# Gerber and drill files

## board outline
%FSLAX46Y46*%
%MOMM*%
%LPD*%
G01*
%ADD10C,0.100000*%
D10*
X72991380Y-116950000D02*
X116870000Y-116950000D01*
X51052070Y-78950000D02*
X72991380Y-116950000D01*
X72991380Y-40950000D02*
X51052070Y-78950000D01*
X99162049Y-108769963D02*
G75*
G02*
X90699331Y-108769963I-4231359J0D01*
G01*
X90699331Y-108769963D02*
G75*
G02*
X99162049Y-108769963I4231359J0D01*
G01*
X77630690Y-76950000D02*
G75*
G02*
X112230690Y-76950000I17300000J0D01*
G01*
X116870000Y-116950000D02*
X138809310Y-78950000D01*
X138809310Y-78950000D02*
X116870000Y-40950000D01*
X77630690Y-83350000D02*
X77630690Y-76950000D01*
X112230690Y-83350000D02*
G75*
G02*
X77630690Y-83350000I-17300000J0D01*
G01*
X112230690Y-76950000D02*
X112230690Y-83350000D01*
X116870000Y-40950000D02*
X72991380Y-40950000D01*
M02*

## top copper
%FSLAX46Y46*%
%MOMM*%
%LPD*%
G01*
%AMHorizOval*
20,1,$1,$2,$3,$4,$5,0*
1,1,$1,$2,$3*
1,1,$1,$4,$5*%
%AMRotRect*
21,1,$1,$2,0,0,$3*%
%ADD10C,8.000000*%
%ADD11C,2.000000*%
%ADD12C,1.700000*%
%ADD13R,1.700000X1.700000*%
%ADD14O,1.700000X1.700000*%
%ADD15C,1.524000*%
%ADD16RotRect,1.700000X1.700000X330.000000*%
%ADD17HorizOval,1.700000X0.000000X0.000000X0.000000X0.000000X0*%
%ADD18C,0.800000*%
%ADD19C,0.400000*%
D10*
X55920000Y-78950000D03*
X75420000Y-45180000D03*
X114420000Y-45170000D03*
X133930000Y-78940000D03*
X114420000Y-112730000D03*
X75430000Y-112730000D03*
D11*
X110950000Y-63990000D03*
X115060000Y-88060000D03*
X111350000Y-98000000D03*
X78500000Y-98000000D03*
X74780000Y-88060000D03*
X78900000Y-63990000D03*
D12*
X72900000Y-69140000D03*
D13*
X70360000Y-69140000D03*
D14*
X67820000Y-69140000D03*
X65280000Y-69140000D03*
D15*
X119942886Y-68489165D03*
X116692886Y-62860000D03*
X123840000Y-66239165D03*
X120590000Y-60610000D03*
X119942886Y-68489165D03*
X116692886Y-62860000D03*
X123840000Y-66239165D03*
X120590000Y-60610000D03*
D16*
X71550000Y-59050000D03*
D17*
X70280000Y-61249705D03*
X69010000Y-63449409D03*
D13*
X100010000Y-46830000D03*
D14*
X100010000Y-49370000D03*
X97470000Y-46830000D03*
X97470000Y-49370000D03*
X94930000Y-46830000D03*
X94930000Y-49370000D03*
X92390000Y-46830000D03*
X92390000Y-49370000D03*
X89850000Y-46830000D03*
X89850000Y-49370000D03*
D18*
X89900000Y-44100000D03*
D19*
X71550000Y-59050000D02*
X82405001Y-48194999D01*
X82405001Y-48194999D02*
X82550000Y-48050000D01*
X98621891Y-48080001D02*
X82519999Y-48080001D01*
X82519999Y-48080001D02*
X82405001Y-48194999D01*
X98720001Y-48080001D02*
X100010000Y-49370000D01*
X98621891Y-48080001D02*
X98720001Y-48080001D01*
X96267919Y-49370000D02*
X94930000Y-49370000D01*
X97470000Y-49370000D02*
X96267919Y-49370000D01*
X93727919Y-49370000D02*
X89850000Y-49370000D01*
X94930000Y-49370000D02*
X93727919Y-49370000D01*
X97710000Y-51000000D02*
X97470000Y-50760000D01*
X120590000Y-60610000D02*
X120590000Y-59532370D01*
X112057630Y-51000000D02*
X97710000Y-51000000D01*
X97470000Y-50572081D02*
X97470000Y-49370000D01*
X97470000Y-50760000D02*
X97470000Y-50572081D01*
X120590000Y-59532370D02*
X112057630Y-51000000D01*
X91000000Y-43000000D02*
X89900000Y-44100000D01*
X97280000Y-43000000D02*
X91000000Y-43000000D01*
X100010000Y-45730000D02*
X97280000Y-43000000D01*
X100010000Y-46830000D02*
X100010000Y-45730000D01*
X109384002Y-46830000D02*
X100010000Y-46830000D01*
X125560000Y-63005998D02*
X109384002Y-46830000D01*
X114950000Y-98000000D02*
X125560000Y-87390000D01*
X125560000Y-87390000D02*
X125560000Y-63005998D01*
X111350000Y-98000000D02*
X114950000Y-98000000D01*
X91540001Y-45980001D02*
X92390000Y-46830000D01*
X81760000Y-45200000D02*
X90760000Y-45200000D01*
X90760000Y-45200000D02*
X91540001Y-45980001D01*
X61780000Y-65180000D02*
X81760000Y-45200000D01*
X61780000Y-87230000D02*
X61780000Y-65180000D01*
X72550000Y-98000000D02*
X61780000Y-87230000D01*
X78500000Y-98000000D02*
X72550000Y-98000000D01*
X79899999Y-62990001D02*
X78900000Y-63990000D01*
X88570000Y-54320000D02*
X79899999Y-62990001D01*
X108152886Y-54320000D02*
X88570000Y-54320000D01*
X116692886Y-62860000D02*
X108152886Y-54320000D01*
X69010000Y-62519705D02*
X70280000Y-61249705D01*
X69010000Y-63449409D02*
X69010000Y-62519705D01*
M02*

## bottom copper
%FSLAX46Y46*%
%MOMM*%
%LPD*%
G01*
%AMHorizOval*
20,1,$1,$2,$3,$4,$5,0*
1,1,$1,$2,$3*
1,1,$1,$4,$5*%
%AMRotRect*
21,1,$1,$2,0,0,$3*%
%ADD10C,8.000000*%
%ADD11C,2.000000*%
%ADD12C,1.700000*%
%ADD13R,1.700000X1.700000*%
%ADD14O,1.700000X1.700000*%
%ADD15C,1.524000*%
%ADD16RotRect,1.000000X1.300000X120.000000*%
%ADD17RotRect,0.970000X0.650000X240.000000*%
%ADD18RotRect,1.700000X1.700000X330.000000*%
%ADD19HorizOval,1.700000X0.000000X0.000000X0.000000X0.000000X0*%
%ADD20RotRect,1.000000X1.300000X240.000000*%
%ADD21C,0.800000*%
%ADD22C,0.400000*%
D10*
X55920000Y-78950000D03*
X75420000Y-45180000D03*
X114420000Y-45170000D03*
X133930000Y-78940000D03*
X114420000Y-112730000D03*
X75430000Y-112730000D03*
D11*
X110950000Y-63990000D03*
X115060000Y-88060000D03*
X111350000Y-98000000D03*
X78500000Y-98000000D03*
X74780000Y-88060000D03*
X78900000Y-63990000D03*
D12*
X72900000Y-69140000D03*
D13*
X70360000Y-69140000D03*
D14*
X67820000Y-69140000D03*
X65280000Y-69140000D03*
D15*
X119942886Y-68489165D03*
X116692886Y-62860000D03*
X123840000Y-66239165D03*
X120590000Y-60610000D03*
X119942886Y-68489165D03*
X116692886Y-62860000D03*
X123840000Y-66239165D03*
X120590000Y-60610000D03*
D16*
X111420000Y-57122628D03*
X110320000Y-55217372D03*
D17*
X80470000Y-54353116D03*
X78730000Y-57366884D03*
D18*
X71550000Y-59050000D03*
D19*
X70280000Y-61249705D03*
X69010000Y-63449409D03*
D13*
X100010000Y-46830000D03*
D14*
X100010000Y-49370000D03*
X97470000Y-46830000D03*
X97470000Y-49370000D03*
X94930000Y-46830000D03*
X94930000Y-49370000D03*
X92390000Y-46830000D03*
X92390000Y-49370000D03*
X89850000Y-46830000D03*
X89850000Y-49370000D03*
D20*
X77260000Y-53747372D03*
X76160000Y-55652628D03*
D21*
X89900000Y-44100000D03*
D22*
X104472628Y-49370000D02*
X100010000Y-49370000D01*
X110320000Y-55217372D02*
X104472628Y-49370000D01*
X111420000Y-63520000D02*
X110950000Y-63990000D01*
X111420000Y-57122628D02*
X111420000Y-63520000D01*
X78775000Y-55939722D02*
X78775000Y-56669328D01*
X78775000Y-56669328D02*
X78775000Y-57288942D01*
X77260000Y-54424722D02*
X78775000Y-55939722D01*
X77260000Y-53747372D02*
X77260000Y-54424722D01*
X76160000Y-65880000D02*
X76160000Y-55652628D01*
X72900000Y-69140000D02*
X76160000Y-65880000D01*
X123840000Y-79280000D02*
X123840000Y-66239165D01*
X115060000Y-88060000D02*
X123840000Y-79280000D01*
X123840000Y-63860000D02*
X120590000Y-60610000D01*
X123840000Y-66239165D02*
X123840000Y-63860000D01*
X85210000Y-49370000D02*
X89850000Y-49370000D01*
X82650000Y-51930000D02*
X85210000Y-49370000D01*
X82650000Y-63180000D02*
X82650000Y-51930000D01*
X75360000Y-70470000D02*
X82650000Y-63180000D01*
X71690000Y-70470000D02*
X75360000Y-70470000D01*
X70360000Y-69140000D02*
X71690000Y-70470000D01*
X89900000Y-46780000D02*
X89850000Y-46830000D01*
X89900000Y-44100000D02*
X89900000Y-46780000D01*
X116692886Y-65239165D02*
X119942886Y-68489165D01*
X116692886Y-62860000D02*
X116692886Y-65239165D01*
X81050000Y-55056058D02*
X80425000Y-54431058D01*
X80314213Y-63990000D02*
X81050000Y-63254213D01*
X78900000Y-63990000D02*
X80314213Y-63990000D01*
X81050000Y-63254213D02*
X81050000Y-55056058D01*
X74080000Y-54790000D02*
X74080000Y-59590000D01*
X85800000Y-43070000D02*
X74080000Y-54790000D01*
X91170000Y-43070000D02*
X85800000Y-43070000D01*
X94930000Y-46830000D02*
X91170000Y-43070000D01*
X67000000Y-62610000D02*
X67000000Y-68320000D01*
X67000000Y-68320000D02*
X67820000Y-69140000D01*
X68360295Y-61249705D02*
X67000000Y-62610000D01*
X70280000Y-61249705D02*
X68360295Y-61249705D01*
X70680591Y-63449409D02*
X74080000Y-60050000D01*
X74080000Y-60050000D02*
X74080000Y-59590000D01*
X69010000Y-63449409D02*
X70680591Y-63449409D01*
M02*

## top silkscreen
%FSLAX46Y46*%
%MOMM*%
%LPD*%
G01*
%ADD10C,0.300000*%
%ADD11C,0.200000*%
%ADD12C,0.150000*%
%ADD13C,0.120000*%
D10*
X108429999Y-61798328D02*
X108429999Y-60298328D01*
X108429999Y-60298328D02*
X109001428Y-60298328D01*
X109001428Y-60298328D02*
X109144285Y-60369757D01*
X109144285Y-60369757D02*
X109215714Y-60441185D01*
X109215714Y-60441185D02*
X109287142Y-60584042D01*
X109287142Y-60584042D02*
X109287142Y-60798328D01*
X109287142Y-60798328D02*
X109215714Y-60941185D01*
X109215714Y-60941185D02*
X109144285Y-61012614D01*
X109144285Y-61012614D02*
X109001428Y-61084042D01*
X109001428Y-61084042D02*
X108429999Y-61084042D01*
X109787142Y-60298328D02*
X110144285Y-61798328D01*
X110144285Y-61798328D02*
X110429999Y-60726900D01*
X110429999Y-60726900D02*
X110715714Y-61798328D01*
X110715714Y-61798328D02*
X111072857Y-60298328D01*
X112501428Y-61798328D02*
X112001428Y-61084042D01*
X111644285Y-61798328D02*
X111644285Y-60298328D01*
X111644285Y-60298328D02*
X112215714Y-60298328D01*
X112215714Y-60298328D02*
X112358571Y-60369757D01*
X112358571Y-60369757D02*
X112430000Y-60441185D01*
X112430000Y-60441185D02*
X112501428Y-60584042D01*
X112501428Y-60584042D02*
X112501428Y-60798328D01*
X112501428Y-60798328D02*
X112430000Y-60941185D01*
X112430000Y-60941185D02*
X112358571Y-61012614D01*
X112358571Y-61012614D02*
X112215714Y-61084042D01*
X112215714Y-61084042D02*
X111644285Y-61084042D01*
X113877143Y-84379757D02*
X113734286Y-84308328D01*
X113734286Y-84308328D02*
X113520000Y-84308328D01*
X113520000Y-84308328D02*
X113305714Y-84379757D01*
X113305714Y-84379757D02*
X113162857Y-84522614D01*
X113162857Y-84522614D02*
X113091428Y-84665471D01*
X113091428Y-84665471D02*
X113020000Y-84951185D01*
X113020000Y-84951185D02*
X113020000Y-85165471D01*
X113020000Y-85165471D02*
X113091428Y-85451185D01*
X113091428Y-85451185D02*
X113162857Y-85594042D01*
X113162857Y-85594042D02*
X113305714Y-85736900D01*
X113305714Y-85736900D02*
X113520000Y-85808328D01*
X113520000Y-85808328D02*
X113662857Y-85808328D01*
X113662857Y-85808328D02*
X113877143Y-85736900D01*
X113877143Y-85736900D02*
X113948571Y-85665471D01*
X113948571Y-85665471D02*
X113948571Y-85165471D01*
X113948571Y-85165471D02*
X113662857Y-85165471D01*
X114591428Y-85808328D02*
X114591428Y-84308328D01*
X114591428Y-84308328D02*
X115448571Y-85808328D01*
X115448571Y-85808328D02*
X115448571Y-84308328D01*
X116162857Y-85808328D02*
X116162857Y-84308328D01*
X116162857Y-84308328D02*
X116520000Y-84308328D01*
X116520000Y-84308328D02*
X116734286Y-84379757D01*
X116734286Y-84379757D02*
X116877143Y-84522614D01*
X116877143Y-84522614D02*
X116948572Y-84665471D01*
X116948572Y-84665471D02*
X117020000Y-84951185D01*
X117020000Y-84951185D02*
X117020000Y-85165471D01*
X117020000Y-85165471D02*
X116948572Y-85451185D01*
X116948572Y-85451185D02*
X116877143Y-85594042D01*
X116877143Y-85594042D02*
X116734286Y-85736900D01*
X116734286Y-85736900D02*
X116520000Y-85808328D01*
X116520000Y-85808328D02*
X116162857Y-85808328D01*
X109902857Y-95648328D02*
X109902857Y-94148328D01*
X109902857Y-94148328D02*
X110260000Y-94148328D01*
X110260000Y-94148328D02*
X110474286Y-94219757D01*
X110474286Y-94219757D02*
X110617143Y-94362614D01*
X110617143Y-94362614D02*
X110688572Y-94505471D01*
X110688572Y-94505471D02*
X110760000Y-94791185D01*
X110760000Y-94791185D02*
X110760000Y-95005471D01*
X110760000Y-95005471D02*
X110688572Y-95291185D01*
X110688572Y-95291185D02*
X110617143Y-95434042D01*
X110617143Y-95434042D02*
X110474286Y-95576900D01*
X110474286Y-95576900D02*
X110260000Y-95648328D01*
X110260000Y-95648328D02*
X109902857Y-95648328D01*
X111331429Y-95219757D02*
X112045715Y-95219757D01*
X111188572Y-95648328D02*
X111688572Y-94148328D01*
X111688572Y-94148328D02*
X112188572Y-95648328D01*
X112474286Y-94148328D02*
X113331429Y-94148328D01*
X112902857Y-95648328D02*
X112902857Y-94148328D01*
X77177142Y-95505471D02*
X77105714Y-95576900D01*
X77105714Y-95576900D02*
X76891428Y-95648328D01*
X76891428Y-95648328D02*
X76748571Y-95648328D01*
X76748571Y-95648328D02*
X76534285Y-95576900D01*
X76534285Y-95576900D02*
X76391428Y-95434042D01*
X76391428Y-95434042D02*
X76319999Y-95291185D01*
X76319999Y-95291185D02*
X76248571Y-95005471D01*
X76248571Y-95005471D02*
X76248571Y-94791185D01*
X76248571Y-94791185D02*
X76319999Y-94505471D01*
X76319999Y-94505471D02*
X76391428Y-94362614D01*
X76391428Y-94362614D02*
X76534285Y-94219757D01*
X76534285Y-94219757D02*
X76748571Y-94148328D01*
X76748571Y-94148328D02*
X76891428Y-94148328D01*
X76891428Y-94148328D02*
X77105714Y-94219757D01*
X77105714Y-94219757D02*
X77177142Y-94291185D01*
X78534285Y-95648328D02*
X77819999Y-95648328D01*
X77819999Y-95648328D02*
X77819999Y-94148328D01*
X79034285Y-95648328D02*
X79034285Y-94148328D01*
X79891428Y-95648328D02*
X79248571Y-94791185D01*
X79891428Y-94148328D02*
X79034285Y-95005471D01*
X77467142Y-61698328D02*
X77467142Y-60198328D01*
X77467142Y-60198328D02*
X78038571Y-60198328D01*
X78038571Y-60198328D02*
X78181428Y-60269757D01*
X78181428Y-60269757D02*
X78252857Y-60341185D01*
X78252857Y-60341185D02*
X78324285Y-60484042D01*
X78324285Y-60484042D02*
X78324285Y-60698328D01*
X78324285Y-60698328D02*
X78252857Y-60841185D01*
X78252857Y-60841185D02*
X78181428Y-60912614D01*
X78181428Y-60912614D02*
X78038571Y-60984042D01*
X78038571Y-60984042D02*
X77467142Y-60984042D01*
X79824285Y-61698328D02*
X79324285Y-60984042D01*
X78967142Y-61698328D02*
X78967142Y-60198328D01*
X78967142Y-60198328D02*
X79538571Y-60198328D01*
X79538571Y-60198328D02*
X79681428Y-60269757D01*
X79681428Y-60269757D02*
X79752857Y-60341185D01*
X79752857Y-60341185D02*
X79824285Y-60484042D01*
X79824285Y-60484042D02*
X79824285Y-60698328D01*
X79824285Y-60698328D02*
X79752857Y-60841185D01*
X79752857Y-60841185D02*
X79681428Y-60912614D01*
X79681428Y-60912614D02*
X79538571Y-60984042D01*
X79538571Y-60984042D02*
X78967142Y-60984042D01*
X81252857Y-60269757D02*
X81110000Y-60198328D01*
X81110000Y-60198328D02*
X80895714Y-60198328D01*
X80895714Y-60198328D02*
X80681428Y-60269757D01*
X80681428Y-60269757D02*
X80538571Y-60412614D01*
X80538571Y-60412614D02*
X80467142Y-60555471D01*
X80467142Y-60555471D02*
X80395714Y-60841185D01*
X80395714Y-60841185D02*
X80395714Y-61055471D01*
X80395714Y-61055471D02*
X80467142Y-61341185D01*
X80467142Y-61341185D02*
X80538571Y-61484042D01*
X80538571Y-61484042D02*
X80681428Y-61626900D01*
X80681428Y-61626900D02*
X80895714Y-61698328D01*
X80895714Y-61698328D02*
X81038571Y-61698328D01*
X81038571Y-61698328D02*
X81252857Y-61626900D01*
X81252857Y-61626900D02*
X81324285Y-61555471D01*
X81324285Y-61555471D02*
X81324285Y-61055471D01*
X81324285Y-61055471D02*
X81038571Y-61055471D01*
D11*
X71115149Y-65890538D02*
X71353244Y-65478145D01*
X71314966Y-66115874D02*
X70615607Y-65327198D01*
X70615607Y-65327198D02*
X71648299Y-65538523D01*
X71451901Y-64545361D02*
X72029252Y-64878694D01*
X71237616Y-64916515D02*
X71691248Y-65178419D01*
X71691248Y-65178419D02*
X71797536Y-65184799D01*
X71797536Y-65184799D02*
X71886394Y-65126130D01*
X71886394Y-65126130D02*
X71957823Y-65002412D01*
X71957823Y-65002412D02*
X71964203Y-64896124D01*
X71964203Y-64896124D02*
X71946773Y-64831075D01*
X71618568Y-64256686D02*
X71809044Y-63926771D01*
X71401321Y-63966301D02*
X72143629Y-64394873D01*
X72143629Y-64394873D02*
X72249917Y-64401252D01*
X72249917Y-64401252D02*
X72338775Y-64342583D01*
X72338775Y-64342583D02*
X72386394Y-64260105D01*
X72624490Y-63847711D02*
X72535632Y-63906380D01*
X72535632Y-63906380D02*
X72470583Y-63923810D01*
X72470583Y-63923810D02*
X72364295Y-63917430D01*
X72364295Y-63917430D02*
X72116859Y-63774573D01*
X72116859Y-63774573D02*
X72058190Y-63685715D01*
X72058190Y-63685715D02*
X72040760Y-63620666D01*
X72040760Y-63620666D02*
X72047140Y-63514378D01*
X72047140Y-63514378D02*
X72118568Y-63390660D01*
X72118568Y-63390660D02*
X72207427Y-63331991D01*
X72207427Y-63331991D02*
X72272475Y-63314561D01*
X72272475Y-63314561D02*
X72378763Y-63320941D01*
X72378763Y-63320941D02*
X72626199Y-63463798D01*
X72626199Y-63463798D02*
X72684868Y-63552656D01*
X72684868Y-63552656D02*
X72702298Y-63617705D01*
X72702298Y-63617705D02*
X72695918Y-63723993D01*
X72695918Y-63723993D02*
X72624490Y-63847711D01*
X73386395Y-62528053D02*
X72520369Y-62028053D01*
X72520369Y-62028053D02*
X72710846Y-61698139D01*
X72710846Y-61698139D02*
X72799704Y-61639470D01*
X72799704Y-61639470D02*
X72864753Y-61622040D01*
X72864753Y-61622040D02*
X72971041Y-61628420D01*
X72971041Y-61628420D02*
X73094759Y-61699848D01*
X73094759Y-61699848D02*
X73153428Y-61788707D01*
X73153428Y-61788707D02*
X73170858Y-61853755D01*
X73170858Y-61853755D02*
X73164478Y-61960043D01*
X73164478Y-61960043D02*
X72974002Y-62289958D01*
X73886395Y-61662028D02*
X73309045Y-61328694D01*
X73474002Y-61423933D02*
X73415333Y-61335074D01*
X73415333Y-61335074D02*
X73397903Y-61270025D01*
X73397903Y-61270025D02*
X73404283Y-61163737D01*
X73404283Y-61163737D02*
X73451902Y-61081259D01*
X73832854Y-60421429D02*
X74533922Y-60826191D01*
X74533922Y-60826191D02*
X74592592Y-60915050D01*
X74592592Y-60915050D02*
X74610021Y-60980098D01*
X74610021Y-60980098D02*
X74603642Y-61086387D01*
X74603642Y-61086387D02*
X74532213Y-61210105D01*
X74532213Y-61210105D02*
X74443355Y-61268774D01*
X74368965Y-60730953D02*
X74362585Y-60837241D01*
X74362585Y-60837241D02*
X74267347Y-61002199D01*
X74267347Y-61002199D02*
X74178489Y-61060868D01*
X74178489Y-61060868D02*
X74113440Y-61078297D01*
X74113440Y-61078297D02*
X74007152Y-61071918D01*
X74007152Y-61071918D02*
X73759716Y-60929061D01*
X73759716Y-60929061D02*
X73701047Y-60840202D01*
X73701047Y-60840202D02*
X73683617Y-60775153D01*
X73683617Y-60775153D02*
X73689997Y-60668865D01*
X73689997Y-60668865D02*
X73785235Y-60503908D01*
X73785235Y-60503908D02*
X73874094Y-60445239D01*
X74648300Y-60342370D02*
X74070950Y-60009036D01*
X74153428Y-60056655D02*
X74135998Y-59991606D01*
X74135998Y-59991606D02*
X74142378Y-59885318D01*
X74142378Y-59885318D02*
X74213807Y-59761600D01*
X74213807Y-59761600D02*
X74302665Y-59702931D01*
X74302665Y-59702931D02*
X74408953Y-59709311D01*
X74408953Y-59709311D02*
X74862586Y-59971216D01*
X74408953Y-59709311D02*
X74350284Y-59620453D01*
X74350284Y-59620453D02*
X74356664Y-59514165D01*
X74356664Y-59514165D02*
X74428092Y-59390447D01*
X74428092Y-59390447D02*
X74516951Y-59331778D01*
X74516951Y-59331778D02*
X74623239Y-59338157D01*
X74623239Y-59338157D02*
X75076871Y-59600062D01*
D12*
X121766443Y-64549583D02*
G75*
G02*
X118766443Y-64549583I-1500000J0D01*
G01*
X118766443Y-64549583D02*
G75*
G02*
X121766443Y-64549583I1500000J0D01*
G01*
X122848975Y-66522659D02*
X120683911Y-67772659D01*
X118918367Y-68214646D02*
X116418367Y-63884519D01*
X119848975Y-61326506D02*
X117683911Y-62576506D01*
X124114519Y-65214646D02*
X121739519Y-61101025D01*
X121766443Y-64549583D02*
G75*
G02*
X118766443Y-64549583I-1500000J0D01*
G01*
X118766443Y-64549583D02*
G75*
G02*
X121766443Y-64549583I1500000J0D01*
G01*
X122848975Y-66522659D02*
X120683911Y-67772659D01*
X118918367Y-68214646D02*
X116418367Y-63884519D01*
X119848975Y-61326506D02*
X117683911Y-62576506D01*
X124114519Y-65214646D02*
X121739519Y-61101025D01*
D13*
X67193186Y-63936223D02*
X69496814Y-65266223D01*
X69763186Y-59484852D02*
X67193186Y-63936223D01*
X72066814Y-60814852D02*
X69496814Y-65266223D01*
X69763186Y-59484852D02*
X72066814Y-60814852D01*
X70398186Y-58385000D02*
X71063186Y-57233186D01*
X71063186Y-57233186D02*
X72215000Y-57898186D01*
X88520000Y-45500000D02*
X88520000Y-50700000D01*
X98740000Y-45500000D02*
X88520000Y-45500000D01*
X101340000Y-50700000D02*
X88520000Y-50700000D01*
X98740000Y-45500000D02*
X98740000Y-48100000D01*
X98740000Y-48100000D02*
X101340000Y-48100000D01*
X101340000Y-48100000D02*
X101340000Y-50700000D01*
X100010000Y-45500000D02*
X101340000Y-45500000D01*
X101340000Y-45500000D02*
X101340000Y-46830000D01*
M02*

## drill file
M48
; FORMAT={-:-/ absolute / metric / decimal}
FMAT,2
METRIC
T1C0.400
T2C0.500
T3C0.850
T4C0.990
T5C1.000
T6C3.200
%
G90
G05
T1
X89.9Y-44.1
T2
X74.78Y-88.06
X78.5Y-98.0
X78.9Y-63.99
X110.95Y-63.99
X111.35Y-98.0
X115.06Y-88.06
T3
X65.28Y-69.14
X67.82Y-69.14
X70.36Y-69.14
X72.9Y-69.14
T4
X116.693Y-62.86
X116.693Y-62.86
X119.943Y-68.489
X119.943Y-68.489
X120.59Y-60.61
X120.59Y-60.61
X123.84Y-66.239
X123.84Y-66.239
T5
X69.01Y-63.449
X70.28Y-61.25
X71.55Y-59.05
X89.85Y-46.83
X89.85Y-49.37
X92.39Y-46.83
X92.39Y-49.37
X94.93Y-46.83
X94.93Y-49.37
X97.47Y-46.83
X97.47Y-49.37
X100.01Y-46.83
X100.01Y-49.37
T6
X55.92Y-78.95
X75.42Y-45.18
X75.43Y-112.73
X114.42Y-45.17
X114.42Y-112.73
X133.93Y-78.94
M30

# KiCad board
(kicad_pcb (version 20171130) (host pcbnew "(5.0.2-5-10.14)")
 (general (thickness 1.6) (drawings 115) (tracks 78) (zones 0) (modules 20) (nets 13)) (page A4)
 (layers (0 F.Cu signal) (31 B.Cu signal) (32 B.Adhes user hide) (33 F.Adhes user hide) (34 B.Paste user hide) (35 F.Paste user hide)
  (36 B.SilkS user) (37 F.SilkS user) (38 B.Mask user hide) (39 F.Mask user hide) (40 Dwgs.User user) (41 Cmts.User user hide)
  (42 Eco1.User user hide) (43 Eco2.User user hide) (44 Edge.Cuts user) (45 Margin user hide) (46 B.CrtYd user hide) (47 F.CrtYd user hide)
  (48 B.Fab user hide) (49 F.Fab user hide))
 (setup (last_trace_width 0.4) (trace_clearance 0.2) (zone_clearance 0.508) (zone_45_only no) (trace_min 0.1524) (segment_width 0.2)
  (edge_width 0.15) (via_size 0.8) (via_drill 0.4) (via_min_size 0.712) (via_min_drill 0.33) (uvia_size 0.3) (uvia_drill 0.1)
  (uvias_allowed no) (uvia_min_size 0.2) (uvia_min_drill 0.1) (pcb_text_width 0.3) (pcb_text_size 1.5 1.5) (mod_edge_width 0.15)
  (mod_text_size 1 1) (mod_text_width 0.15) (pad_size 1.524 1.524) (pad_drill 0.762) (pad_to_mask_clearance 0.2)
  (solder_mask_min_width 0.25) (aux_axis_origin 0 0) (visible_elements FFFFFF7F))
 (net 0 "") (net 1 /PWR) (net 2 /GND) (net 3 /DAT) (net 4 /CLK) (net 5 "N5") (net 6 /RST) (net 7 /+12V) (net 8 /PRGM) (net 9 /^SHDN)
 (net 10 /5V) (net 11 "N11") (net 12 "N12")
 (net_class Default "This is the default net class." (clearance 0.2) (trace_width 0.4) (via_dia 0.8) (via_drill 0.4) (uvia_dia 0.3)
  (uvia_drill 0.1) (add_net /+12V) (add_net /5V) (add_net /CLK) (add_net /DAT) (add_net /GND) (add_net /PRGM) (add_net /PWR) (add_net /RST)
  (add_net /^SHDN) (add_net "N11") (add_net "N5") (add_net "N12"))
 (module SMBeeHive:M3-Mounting (layer F.Cu) (at 55.92 78.95)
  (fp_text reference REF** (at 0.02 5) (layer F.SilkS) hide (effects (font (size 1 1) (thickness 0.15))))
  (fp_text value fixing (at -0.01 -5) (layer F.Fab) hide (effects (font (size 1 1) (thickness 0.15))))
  (pad "" np_thru_hole circle (at 0 0) (size 8 8) (drill 3.2) (layers *.Cu)))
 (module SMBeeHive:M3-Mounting (layer F.Cu) (at 75.42 45.18)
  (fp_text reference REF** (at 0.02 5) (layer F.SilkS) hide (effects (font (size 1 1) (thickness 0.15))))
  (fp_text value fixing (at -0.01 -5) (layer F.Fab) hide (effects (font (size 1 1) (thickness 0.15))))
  (pad "" np_thru_hole circle (at 0 0) (size 8 8) (drill 3.2) (layers *.Cu)))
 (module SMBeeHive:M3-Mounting (layer F.Cu) (at 114.42 45.17)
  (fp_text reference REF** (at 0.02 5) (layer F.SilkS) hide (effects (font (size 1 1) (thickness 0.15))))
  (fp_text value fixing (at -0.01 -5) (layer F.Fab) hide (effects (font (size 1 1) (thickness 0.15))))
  (pad "" np_thru_hole circle (at 0 0) (size 8 8) (drill 3.2) (layers *.Cu)))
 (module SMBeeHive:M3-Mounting (layer F.Cu) (at 133.93 78.94)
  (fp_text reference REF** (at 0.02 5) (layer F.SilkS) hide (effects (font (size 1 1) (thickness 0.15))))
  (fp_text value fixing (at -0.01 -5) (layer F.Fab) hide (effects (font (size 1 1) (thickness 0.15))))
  (pad "" np_thru_hole circle (at 0 0) (size 8 8) (drill 3.2) (layers *.Cu)))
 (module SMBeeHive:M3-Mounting (layer F.Cu) (at 114.42 112.73)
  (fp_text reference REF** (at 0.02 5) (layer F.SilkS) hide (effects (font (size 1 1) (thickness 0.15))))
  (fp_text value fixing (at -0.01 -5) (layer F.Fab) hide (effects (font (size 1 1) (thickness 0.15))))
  (pad "" np_thru_hole circle (at 0 0) (size 8 8) (drill 3.2) (layers *.Cu)))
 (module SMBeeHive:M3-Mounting (layer F.Cu) (at 75.43 112.73)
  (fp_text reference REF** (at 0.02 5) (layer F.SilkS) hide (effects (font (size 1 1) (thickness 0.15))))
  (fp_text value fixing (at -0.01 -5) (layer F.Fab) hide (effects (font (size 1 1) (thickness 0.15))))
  (pad "" np_thru_hole circle (at 0 0) (size 8 8) (drill 3.2) (layers *.Cu)))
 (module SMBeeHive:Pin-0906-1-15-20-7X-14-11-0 (layer F.Cu) (at 110.95 63.99)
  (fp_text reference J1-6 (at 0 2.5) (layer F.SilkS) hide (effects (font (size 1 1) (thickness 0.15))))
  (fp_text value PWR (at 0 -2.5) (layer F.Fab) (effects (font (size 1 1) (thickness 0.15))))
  (pad 1 thru_hole circle (at 0 0) (size 2 2) (drill 0.5) (layers *.Cu *.Mask) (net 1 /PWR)))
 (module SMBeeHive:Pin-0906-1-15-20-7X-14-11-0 (layer F.Cu) (at 115.06 88.06)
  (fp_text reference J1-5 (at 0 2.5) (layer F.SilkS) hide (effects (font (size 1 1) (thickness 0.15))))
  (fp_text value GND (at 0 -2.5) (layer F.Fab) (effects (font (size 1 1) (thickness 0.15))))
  (pad 1 thru_hole circle (at 0 0) (size 2 2) (drill 0.5) (layers *.Cu *.Mask) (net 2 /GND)))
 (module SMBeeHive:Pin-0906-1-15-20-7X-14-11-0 (layer F.Cu) (at 111.35 98)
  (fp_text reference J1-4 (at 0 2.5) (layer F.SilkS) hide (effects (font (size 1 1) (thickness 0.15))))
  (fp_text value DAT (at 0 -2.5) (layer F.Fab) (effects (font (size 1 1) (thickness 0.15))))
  (pad 1 thru_hole circle (at 0 0) (size 2 2) (drill 0.5) (layers *.Cu *.Mask) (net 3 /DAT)))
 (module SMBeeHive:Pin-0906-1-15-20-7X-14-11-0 (layer F.Cu) (at 78.5 98)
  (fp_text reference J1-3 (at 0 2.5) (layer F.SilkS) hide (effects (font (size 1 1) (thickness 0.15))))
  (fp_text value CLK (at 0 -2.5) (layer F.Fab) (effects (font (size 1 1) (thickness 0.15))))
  (pad 1 thru_hole circle (at 0 0) (size 2 2) (drill 0.5) (layers *.Cu *.Mask) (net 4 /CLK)))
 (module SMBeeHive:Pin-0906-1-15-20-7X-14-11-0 (layer F.Cu) (at 74.78 88.06)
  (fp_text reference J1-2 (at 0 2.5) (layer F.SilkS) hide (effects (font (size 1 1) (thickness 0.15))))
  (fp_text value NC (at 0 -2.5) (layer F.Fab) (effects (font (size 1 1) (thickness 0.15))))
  (pad 1 thru_hole circle (at 0 0) (size 2 2) (drill 0.5) (layers *.Cu *.Mask) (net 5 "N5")))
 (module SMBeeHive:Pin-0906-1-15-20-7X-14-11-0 (layer F.Cu) (at 78.9 63.99)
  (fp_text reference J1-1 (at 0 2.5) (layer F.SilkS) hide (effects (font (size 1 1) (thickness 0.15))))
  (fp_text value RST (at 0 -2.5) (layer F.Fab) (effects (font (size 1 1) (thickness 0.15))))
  (pad 1 thru_hole circle (at 0 0) (size 2 2) (drill 0.5) (layers *.Cu *.Mask) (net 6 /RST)))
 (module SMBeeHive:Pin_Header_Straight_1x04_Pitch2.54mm (layer B.Cu) (at 72.9 69.14 90)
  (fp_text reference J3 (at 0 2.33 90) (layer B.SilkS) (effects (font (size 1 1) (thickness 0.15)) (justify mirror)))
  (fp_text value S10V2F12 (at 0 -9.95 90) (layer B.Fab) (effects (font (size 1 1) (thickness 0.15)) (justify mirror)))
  (pad 1 thru_hole circle (at 0 0 90) (size 1.7 1.7) (drill 0.85) (layers *.Cu *.Mask) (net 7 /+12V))
  (pad 2 thru_hole rect (at 0 -2.54 90) (size 1.7 1.7) (drill 0.85) (layers *.Cu *.Mask) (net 2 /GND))
  (pad 3 thru_hole oval (at 0 -5.08 90) (size 1.7 1.7) (drill 0.85) (layers *.Cu *.Mask) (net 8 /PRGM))
  (pad 4 thru_hole oval (at 0 -7.62 90) (size 1.7 1.7) (drill 0.85) (layers *.Cu *.Mask) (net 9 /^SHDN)))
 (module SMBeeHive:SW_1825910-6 (layer F.Cu) (at 120.59 60.61 300)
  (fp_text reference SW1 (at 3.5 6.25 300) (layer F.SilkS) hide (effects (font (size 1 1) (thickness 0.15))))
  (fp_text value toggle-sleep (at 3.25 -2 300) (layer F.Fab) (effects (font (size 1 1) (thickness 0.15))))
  (fp_circle (center 3.25 2.25) (end 4.75 2.25) (layer F.SilkS) (width 0.15))
  (fp_line (start 6.25 1) (end 6.25 3.5) (layer F.SilkS) (width 0.15))
  (fp_line (start 5.75 5.25) (end 0.75 5.25) (layer F.SilkS) (width 0.15))
  (fp_line (start 0.25 0.999999) (end 0.25 3.5) (layer F.SilkS) (width 0.15))
  (fp_line (start 5.75 -0.75) (end 1 -0.75) (layer F.SilkS) (width 0.15))
  (pad 4 thru_hole circle (at 6.5 4.5 300) (size 1.524 1.524) (drill 0.99) (layers *.Cu *.Mask) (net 6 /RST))
  (pad 3 thru_hole circle (at 0 4.5 300) (size 1.524 1.524) (drill 0.99) (layers *.Cu *.Mask) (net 6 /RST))
  (pad 2 thru_hole circle (at 6.5 0 300) (size 1.524 1.524) (drill 0.99) (layers *.Cu *.Mask) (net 2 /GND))
  (pad 1 thru_hole circle (at 0 0 300) (size 1.524 1.524) (drill 0.99) (layers *.Cu *.Mask) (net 2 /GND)))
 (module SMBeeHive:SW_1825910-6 (layer F.Cu) (at 120.59 60.61 300)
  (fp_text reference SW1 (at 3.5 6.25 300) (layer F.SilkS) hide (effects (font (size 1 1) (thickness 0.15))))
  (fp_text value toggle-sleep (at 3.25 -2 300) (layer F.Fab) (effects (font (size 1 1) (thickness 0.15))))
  (fp_circle (center 3.25 2.25) (end 4.75 2.25) (layer F.SilkS) (width 0.15))
  (fp_line (start 6.25 1) (end 6.25 3.5) (layer F.SilkS) (width 0.15))
  (fp_line (start 5.75 5.25) (end 0.75 5.25) (layer F.SilkS) (width 0.15))
  (fp_line (start 0.25 0.999999) (end 0.25 3.5) (layer F.SilkS) (width 0.15))
  (fp_line (start 5.75 -0.75) (end 1 -0.75) (layer F.SilkS) (width 0.15))
  (pad 4 thru_hole circle (at 6.5 4.5 300) (size 1.524 1.524) (drill 0.99) (layers *.Cu *.Mask) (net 6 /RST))
  (pad 3 thru_hole circle (at 0 4.5 300) (size 1.524 1.524) (drill 0.99) (layers *.Cu *.Mask) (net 6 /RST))
  (pad 2 thru_hole circle (at 6.5 0 300) (size 1.524 1.524) (drill 0.99) (layers *.Cu *.Mask) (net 2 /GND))
  (pad 1 thru_hole circle (at 0 0 300) (size 1.524 1.524) (drill 0.99) (layers *.Cu *.Mask) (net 2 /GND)))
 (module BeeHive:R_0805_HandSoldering (layer B.Cu) (at 110.87 56.17 120)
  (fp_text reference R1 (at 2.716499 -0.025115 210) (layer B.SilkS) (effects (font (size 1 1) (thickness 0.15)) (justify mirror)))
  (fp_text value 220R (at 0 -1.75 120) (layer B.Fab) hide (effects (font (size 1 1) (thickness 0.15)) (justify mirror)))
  (pad 1 smd rect (at -1.1 0 120) (size 1 1.3) (layers B.Cu B.Paste B.Mask) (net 1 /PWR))
  (pad 2 smd rect (at 1.1 0 120) (size 1 1.3) (layers B.Cu B.Paste B.Mask) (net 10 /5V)))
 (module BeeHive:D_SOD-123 (layer B.Cu) (at 79.6 55.86 240)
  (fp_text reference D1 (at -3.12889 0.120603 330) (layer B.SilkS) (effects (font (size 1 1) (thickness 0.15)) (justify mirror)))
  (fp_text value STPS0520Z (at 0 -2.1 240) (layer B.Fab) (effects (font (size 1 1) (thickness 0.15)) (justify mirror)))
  (pad 1 smd rect (at -1.74 0 240) (size 0.97 0.65) (layers B.Cu B.Paste B.Mask) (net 6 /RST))
  (pad 2 smd rect (at 1.74 0 240) (size 0.97 0.65) (layers B.Cu B.Paste B.Mask) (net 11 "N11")))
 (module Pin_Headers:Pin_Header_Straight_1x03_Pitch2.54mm (layer F.Cu) (at 71.55 59.05 330)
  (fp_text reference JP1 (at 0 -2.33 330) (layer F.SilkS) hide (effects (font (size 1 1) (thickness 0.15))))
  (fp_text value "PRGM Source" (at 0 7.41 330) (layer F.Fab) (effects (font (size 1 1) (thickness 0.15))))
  (fp_line (start -1.33 6.41) (end 1.33 6.41) (layer F.SilkS) (width 0.12))
  (fp_line (start -1.33 1.27) (end -1.33 6.41) (layer F.SilkS) (width 0.12))
  (fp_line (start 1.33 1.27) (end 1.33 6.41) (layer F.SilkS) (width 0.12))
  (fp_line (start -1.33 1.27) (end 1.33 1.27) (layer F.SilkS) (width 0.12))
  (fp_line (start -1.33 0) (end -1.33 -1.33) (layer F.SilkS) (width 0.12))
  (fp_line (start -1.33 -1.33) (end 0 -1.33) (layer F.SilkS) (width 0.12))
  (pad 1 thru_hole rect (at 0 0 330) (size 1.7 1.7) (drill 1) (layers *.Cu *.Mask) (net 10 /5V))
  (pad 2 thru_hole oval (at 0 2.54 330) (size 1.7 1.7) (drill 1) (layers *.Cu *.Mask) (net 8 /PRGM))
  (pad 3 thru_hole oval (at 0 5.08 330) (size 1.7 1.7) (drill 1) (layers *.Cu *.Mask) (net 8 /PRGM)))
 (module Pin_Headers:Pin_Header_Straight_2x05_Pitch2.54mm (layer F.Cu) (at 100.01 46.83 270)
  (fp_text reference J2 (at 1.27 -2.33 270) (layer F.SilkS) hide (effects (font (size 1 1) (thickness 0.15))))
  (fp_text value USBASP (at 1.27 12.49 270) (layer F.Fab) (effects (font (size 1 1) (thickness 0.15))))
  (fp_line (start -1.33 11.49) (end 3.87 11.49) (layer F.SilkS) (width 0.12))
  (fp_line (start -1.33 1.27) (end -1.33 11.49) (layer F.SilkS) (width 0.12))
  (fp_line (start 3.87 -1.33) (end 3.87 11.49) (layer F.SilkS) (width 0.12))
  (fp_line (start -1.33 1.27) (end 1.27 1.27) (layer F.SilkS) (width 0.12))
  (fp_line (start 1.27 1.27) (end 1.27 -1.33) (layer F.SilkS) (width 0.12))
  (fp_line (start 1.27 -1.33) (end 3.87 -1.33) (layer F.SilkS) (width 0.12))
  (fp_line (start -1.33 0) (end -1.33 -1.33) (layer F.SilkS) (width 0.12))
  (fp_line (start -1.33 -1.33) (end 0 -1.33) (layer F.SilkS) (width 0.12))
  (pad 1 thru_hole rect (at 0 0 270) (size 1.7 1.7) (drill 1) (layers *.Cu *.Mask) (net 3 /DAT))
  (pad 2 thru_hole oval (at 2.54 0 270) (size 1.7 1.7) (drill 1) (layers *.Cu *.Mask) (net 10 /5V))
  (pad 3 thru_hole oval (at 0 2.54 270) (size 1.7 1.7) (drill 1) (layers *.Cu *.Mask) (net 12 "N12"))
  (pad 4 thru_hole oval (at 2.54 2.54 270) (size 1.7 1.7) (drill 1) (layers *.Cu *.Mask) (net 2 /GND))
  (pad 5 thru_hole oval (at 0 5.08 270) (size 1.7 1.7) (drill 1) (layers *.Cu *.Mask) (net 8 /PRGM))
  (pad 6 thru_hole oval (at 2.54 5.08 270) (size 1.7 1.7) (drill 1) (layers *.Cu *.Mask) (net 2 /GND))
  (pad 7 thru_hole oval (at 0 7.62 270) (size 1.7 1.7) (drill 1) (layers *.Cu *.Mask) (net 4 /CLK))
  (pad 8 thru_hole oval (at 2.54 7.62 270) (size 1.7 1.7) (drill 1) (layers *.Cu *.Mask) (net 2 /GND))
  (pad 9 thru_hole oval (at 0 10.16 270) (size 1.7 1.7) (drill 1) (layers *.Cu *.Mask) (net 3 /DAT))
  (pad 10 thru_hole oval (at 2.54 10.16 270) (size 1.7 1.7) (drill 1) (layers *.Cu *.Mask) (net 2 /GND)))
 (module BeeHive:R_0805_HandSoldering (layer B.Cu) (at 76.71 54.7 240)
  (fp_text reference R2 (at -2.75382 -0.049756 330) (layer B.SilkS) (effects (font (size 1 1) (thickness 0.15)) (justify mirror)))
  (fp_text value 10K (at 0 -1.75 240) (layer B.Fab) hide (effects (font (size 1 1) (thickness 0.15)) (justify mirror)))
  (pad 1 smd rect (at -1.1 0 240) (size 1 1.3) (layers B.Cu B.Paste B.Mask) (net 11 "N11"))
  (pad 2 smd rect (at 1.1 0 240) (size 1 1.3) (layers B.Cu B.Paste B.Mask) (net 7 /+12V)))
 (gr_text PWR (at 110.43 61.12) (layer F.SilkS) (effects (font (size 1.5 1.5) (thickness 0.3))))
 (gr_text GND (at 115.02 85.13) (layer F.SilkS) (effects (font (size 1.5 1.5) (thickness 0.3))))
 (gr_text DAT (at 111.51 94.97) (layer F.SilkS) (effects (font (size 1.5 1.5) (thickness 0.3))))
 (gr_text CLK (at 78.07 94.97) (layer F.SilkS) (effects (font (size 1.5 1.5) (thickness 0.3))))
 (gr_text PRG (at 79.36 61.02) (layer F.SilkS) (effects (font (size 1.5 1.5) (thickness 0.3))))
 (gr_line (start 72.99138 116.95) (end 116.87 116.95) (layer Edge.Cuts) (width 0.1))
 (gr_line (start 51.05207 78.95) (end 72.99138 116.95) (layer Edge.Cuts) (width 0.1))
 (gr_line (start 72.99138 40.95) (end 51.05207 78.95) (layer Edge.Cuts) (width 0.1))
 (gr_circle (center 94.93069 108.769963) (end 99.162049 108.769963) (layer Edge.Cuts) (width 0.1))
 (gr_arc (start 94.93069 76.95) (end 112.23069 76.95) (angle -180) (layer Edge.Cuts) (width 0.1))
 (gr_line (start 116.87 116.95) (end 138.80931 78.95) (layer Edge.Cuts) (width 0.1))
 (gr_line (start 138.80931 78.95) (end 116.87 40.95) (layer Edge.Cuts) (width 0.1))
 (gr_line (start 77.63069 83.35) (end 77.63069 76.95) (layer Edge.Cuts) (width 0.1))
 (gr_arc (start 94.93069 83.35) (end 77.63069 83.35) (angle -180) (layer Edge.Cuts) (width 0.1))
 (gr_line (start 112.23069 76.95) (end 112.23069 83.35) (layer Edge.Cuts) (width 0.1))
 (gr_line (start 116.87 40.95) (end 72.99138 40.95) (layer Edge.Cuts) (width 0.1))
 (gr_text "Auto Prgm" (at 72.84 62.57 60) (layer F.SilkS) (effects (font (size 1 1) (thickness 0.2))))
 (segment (start 104.472628 49.37) (end 100.01 49.37) (width 0.4) (layer B.Cu) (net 10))
 (segment (start 110.32 55.217372) (end 104.472628 49.37) (width 0.4) (layer B.Cu) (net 10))
 (segment (start 71.55 59.05) (end 82.405001 48.194999) (width 0.4) (layer F.Cu) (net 10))
 (segment (start 82.405001 48.194999) (end 82.55 48.05) (width 0.4) (layer F.Cu) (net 10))
 (segment (start 98.621891 48.080001) (end 82.519999 48.080001) (width 0.4) (layer F.Cu) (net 10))
 (segment (start 82.519999 48.080001) (end 82.405001 48.194999) (width 0.4) (layer F.Cu) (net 10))
 (segment (start 98.720001 48.080001) (end 100.01 49.37) (width 0.4) (layer F.Cu) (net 10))
 (segment (start 98.621891 48.080001) (end 98.720001 48.080001) (width 0.4) (layer F.Cu) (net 10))
 (segment (start 111.42 63.52) (end 110.95 63.99) (width 0.4) (layer B.Cu) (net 1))
 (segment (start 111.42 57.122628) (end 111.42 63.52) (width 0.4) (layer B.Cu) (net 1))
 (segment (start 78.775 55.939722) (end 78.775 56.669328) (width 0.4) (layer B.Cu) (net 11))
 (segment (start 78.775 56.669328) (end 78.775 57.288942) (width 0.4) (layer B.Cu) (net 11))
 (segment (start 77.26 54.424722) (end 78.775 55.939722) (width 0.4) (layer B.Cu) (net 11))
 (segment (start 77.26 53.747372) (end 77.26 54.424722) (width 0.4) (layer B.Cu) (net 11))
 (segment (start 76.16 65.88) (end 76.16 55.652628) (width 0.4) (layer B.Cu) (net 7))
 (segment (start 72.9 69.14) (end 76.16 65.88) (width 0.4) (layer B.Cu) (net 7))
 (segment (start 123.84 79.28) (end 123.84 66.239165) (width 0.4) (layer B.Cu) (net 2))
 (segment (start 115.06 88.06) (end 123.84 79.28) (width 0.4) (layer B.Cu) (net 2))
 (segment (start 123.84 63.86) (end 120.59 60.61) (width 0.4) (layer B.Cu) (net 2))
 (segment (start 123.84 66.239165) (end 123.84 63.86) (width 0.4) (layer B.Cu) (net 2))
 (segment (start 96.267919 49.37) (end 94.93 49.37) (width 0.4) (layer F.Cu) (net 2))
 (segment (start 97.47 49.37) (end 96.267919 49.37) (width 0.4) (layer F.Cu) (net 2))
 (segment (start 93.727919 49.37) (end 89.85 49.37) (width 0.4) (layer F.Cu) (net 2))
 (segment (start 94.93 49.37) (end 93.727919 49.37) (width 0.4) (layer F.Cu) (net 2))
 (segment (start 97.71 51) (end 97.47 50.76) (width 0.4) (layer F.Cu) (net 2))
 (segment (start 120.59 60.61) (end 120.59 59.53237) (width 0.4) (layer F.Cu) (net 2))
 (segment (start 112.05763 51) (end 97.71 51) (width 0.4) (layer F.Cu) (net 2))
 (segment (start 97.47 50.572081) (end 97.47 49.37) (width 0.4) (layer F.Cu) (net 2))
 (segment (start 97.47 50.76) (end 97.47 50.572081) (width 0.4) (layer F.Cu) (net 2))
 (segment (start 120.59 59.53237) (end 112.05763 51) (width 0.4) (layer F.Cu) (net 2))
 (segment (start 85.21 49.37) (end 89.85 49.37) (width 0.4) (layer B.Cu) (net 2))
 (segment (start 82.65 51.93) (end 85.21 49.37) (width 0.4) (layer B.Cu) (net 2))
 (segment (start 82.65 63.18) (end 82.65 51.93) (width 0.4) (layer B.Cu) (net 2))
 (segment (start 75.36 70.47) (end 82.65 63.18) (width 0.4) (layer B.Cu) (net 2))
 (segment (start 71.69 70.47) (end 75.36 70.47) (width 0.4) (layer B.Cu) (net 2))
 (segment (start 70.36 69.14) (end 71.69 70.47) (width 0.4) (layer B.Cu) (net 2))
 (via (at 89.9 44.1) (size 0.8) (drill 0.4) (layers F.Cu B.Cu) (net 3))
 (segment (start 89.9 46.78) (end 89.85 46.83) (width 0.4) (layer B.Cu) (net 3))
 (segment (start 89.9 44.1) (end 89.9 46.78) (width 0.4) (layer B.Cu) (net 3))
 (segment (start 91 43) (end 89.9 44.1) (width 0.4) (layer F.Cu) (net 3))
 (segment (start 97.28 43) (end 91 43) (width 0.4) (layer F.Cu) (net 3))
 (segment (start 100.01 45.73) (end 97.28 43) (width 0.4) (layer F.Cu) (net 3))
 (segment (start 100.01 46.83) (end 100.01 45.73) (width 0.4) (layer F.Cu) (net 3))
 (segment (start 109.384002 46.83) (end 100.01 46.83) (width 0.4) (layer F.Cu) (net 3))
 (segment (start 125.56 63.005998) (end 109.384002 46.83) (width 0.4) (layer F.Cu) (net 3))
 (segment (start 114.95 98) (end 125.56 87.39) (width 0.4) (layer F.Cu) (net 3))
 (segment (start 125.56 87.39) (end 125.56 63.005998) (width 0.4) (layer F.Cu) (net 3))
 (segment (start 111.35 98) (end 114.95 98) (width 0.4) (layer F.Cu) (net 3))
 (segment (start 91.540001 45.980001) (end 92.39 46.83) (width 0.4) (layer F.Cu) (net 4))
 (segment (start 81.76 45.2) (end 90.76 45.2) (width 0.4) (layer F.Cu) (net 4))
 (segment (start 90.76 45.2) (end 91.540001 45.980001) (width 0.4) (layer F.Cu) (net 4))
 (segment (start 61.78 65.18) (end 81.76 45.2) (width 0.4) (layer F.Cu) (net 4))
 (segment (start 61.78 87.23) (end 61.78 65.18) (width 0.4) (layer F.Cu) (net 4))
 (segment (start 72.55 98) (end 61.78 87.23) (width 0.4) (layer F.Cu) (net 4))
 (segment (start 78.5 98) (end 72.55 98) (width 0.4) (layer F.Cu) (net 4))
 (segment (start 116.692886 65.239165) (end 119.942886 68.489165) (width 0.4) (layer B.Cu) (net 6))
 (segment (start 116.692886 62.86) (end 116.692886 65.239165) (width 0.4) (layer B.Cu) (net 6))
 (segment (start 79.899999 62.990001) (end 78.9 63.99) (width 0.4) (layer F.Cu) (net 6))
 (segment (start 88.57 54.32) (end 79.899999 62.990001) (width 0.4) (layer F.Cu) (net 6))
 (segment (start 108.152886 54.32) (end 88.57 54.32) (width 0.4) (layer F.Cu) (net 6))
 (segment (start 116.692886 62.86) (end 108.152886 54.32) (width 0.4) (layer F.Cu) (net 6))
 (segment (start 81.05 55.056058) (end 80.425 54.431058) (width 0.4) (layer B.Cu) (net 6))
 (segment (start 80.314213 63.99) (end 81.05 63.254213) (width 0.4) (layer B.Cu) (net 6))
 (segment (start 78.9 63.99) (end 80.314213 63.99) (width 0.4) (layer B.Cu) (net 6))
 (segment (start 81.05 63.254213) (end 81.05 55.056058) (width 0.4) (layer B.Cu) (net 6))
 (segment (start 74.08 54.79) (end 74.08 59.59) (width 0.4) (layer B.Cu) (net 8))
 (segment (start 85.8 43.07) (end 74.08 54.79) (width 0.4) (layer B.Cu) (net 8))
 (segment (start 91.17 43.07) (end 85.8 43.07) (width 0.4) (layer B.Cu) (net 8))
 (segment (start 94.93 46.83) (end 91.17 43.07) (width 0.4) (layer B.Cu) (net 8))
 (segment (start 69.01 62.519705) (end 70.28 61.249705) (width 0.4) (layer F.Cu) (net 8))
 (segment (start 69.01 63.449409) (end 69.01 62.519705) (width 0.4) (layer F.Cu) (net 8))
 (segment (start 67 62.61) (end 67 68.32) (width 0.4) (layer B.Cu) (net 8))
 (segment (start 67 68.32) (end 67.82 69.14) (width 0.4) (layer B.Cu) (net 8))
 (segment (start 68.360295 61.249705) (end 67 62.61) (width 0.4) (layer B.Cu) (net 8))
 (segment (start 70.28 61.249705) (end 68.360295 61.249705) (width 0.4) (layer B.Cu) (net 8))
 (segment (start 70.680591 63.449409) (end 74.08 60.05) (width 0.4) (layer B.Cu) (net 8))
 (segment (start 74.08 60.05) (end 74.08 59.59) (width 0.4) (layer B.Cu) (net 8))
 (segment (start 69.01 63.449409) (end 70.680591 63.449409) (width 0.4) (layer B.Cu) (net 8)))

